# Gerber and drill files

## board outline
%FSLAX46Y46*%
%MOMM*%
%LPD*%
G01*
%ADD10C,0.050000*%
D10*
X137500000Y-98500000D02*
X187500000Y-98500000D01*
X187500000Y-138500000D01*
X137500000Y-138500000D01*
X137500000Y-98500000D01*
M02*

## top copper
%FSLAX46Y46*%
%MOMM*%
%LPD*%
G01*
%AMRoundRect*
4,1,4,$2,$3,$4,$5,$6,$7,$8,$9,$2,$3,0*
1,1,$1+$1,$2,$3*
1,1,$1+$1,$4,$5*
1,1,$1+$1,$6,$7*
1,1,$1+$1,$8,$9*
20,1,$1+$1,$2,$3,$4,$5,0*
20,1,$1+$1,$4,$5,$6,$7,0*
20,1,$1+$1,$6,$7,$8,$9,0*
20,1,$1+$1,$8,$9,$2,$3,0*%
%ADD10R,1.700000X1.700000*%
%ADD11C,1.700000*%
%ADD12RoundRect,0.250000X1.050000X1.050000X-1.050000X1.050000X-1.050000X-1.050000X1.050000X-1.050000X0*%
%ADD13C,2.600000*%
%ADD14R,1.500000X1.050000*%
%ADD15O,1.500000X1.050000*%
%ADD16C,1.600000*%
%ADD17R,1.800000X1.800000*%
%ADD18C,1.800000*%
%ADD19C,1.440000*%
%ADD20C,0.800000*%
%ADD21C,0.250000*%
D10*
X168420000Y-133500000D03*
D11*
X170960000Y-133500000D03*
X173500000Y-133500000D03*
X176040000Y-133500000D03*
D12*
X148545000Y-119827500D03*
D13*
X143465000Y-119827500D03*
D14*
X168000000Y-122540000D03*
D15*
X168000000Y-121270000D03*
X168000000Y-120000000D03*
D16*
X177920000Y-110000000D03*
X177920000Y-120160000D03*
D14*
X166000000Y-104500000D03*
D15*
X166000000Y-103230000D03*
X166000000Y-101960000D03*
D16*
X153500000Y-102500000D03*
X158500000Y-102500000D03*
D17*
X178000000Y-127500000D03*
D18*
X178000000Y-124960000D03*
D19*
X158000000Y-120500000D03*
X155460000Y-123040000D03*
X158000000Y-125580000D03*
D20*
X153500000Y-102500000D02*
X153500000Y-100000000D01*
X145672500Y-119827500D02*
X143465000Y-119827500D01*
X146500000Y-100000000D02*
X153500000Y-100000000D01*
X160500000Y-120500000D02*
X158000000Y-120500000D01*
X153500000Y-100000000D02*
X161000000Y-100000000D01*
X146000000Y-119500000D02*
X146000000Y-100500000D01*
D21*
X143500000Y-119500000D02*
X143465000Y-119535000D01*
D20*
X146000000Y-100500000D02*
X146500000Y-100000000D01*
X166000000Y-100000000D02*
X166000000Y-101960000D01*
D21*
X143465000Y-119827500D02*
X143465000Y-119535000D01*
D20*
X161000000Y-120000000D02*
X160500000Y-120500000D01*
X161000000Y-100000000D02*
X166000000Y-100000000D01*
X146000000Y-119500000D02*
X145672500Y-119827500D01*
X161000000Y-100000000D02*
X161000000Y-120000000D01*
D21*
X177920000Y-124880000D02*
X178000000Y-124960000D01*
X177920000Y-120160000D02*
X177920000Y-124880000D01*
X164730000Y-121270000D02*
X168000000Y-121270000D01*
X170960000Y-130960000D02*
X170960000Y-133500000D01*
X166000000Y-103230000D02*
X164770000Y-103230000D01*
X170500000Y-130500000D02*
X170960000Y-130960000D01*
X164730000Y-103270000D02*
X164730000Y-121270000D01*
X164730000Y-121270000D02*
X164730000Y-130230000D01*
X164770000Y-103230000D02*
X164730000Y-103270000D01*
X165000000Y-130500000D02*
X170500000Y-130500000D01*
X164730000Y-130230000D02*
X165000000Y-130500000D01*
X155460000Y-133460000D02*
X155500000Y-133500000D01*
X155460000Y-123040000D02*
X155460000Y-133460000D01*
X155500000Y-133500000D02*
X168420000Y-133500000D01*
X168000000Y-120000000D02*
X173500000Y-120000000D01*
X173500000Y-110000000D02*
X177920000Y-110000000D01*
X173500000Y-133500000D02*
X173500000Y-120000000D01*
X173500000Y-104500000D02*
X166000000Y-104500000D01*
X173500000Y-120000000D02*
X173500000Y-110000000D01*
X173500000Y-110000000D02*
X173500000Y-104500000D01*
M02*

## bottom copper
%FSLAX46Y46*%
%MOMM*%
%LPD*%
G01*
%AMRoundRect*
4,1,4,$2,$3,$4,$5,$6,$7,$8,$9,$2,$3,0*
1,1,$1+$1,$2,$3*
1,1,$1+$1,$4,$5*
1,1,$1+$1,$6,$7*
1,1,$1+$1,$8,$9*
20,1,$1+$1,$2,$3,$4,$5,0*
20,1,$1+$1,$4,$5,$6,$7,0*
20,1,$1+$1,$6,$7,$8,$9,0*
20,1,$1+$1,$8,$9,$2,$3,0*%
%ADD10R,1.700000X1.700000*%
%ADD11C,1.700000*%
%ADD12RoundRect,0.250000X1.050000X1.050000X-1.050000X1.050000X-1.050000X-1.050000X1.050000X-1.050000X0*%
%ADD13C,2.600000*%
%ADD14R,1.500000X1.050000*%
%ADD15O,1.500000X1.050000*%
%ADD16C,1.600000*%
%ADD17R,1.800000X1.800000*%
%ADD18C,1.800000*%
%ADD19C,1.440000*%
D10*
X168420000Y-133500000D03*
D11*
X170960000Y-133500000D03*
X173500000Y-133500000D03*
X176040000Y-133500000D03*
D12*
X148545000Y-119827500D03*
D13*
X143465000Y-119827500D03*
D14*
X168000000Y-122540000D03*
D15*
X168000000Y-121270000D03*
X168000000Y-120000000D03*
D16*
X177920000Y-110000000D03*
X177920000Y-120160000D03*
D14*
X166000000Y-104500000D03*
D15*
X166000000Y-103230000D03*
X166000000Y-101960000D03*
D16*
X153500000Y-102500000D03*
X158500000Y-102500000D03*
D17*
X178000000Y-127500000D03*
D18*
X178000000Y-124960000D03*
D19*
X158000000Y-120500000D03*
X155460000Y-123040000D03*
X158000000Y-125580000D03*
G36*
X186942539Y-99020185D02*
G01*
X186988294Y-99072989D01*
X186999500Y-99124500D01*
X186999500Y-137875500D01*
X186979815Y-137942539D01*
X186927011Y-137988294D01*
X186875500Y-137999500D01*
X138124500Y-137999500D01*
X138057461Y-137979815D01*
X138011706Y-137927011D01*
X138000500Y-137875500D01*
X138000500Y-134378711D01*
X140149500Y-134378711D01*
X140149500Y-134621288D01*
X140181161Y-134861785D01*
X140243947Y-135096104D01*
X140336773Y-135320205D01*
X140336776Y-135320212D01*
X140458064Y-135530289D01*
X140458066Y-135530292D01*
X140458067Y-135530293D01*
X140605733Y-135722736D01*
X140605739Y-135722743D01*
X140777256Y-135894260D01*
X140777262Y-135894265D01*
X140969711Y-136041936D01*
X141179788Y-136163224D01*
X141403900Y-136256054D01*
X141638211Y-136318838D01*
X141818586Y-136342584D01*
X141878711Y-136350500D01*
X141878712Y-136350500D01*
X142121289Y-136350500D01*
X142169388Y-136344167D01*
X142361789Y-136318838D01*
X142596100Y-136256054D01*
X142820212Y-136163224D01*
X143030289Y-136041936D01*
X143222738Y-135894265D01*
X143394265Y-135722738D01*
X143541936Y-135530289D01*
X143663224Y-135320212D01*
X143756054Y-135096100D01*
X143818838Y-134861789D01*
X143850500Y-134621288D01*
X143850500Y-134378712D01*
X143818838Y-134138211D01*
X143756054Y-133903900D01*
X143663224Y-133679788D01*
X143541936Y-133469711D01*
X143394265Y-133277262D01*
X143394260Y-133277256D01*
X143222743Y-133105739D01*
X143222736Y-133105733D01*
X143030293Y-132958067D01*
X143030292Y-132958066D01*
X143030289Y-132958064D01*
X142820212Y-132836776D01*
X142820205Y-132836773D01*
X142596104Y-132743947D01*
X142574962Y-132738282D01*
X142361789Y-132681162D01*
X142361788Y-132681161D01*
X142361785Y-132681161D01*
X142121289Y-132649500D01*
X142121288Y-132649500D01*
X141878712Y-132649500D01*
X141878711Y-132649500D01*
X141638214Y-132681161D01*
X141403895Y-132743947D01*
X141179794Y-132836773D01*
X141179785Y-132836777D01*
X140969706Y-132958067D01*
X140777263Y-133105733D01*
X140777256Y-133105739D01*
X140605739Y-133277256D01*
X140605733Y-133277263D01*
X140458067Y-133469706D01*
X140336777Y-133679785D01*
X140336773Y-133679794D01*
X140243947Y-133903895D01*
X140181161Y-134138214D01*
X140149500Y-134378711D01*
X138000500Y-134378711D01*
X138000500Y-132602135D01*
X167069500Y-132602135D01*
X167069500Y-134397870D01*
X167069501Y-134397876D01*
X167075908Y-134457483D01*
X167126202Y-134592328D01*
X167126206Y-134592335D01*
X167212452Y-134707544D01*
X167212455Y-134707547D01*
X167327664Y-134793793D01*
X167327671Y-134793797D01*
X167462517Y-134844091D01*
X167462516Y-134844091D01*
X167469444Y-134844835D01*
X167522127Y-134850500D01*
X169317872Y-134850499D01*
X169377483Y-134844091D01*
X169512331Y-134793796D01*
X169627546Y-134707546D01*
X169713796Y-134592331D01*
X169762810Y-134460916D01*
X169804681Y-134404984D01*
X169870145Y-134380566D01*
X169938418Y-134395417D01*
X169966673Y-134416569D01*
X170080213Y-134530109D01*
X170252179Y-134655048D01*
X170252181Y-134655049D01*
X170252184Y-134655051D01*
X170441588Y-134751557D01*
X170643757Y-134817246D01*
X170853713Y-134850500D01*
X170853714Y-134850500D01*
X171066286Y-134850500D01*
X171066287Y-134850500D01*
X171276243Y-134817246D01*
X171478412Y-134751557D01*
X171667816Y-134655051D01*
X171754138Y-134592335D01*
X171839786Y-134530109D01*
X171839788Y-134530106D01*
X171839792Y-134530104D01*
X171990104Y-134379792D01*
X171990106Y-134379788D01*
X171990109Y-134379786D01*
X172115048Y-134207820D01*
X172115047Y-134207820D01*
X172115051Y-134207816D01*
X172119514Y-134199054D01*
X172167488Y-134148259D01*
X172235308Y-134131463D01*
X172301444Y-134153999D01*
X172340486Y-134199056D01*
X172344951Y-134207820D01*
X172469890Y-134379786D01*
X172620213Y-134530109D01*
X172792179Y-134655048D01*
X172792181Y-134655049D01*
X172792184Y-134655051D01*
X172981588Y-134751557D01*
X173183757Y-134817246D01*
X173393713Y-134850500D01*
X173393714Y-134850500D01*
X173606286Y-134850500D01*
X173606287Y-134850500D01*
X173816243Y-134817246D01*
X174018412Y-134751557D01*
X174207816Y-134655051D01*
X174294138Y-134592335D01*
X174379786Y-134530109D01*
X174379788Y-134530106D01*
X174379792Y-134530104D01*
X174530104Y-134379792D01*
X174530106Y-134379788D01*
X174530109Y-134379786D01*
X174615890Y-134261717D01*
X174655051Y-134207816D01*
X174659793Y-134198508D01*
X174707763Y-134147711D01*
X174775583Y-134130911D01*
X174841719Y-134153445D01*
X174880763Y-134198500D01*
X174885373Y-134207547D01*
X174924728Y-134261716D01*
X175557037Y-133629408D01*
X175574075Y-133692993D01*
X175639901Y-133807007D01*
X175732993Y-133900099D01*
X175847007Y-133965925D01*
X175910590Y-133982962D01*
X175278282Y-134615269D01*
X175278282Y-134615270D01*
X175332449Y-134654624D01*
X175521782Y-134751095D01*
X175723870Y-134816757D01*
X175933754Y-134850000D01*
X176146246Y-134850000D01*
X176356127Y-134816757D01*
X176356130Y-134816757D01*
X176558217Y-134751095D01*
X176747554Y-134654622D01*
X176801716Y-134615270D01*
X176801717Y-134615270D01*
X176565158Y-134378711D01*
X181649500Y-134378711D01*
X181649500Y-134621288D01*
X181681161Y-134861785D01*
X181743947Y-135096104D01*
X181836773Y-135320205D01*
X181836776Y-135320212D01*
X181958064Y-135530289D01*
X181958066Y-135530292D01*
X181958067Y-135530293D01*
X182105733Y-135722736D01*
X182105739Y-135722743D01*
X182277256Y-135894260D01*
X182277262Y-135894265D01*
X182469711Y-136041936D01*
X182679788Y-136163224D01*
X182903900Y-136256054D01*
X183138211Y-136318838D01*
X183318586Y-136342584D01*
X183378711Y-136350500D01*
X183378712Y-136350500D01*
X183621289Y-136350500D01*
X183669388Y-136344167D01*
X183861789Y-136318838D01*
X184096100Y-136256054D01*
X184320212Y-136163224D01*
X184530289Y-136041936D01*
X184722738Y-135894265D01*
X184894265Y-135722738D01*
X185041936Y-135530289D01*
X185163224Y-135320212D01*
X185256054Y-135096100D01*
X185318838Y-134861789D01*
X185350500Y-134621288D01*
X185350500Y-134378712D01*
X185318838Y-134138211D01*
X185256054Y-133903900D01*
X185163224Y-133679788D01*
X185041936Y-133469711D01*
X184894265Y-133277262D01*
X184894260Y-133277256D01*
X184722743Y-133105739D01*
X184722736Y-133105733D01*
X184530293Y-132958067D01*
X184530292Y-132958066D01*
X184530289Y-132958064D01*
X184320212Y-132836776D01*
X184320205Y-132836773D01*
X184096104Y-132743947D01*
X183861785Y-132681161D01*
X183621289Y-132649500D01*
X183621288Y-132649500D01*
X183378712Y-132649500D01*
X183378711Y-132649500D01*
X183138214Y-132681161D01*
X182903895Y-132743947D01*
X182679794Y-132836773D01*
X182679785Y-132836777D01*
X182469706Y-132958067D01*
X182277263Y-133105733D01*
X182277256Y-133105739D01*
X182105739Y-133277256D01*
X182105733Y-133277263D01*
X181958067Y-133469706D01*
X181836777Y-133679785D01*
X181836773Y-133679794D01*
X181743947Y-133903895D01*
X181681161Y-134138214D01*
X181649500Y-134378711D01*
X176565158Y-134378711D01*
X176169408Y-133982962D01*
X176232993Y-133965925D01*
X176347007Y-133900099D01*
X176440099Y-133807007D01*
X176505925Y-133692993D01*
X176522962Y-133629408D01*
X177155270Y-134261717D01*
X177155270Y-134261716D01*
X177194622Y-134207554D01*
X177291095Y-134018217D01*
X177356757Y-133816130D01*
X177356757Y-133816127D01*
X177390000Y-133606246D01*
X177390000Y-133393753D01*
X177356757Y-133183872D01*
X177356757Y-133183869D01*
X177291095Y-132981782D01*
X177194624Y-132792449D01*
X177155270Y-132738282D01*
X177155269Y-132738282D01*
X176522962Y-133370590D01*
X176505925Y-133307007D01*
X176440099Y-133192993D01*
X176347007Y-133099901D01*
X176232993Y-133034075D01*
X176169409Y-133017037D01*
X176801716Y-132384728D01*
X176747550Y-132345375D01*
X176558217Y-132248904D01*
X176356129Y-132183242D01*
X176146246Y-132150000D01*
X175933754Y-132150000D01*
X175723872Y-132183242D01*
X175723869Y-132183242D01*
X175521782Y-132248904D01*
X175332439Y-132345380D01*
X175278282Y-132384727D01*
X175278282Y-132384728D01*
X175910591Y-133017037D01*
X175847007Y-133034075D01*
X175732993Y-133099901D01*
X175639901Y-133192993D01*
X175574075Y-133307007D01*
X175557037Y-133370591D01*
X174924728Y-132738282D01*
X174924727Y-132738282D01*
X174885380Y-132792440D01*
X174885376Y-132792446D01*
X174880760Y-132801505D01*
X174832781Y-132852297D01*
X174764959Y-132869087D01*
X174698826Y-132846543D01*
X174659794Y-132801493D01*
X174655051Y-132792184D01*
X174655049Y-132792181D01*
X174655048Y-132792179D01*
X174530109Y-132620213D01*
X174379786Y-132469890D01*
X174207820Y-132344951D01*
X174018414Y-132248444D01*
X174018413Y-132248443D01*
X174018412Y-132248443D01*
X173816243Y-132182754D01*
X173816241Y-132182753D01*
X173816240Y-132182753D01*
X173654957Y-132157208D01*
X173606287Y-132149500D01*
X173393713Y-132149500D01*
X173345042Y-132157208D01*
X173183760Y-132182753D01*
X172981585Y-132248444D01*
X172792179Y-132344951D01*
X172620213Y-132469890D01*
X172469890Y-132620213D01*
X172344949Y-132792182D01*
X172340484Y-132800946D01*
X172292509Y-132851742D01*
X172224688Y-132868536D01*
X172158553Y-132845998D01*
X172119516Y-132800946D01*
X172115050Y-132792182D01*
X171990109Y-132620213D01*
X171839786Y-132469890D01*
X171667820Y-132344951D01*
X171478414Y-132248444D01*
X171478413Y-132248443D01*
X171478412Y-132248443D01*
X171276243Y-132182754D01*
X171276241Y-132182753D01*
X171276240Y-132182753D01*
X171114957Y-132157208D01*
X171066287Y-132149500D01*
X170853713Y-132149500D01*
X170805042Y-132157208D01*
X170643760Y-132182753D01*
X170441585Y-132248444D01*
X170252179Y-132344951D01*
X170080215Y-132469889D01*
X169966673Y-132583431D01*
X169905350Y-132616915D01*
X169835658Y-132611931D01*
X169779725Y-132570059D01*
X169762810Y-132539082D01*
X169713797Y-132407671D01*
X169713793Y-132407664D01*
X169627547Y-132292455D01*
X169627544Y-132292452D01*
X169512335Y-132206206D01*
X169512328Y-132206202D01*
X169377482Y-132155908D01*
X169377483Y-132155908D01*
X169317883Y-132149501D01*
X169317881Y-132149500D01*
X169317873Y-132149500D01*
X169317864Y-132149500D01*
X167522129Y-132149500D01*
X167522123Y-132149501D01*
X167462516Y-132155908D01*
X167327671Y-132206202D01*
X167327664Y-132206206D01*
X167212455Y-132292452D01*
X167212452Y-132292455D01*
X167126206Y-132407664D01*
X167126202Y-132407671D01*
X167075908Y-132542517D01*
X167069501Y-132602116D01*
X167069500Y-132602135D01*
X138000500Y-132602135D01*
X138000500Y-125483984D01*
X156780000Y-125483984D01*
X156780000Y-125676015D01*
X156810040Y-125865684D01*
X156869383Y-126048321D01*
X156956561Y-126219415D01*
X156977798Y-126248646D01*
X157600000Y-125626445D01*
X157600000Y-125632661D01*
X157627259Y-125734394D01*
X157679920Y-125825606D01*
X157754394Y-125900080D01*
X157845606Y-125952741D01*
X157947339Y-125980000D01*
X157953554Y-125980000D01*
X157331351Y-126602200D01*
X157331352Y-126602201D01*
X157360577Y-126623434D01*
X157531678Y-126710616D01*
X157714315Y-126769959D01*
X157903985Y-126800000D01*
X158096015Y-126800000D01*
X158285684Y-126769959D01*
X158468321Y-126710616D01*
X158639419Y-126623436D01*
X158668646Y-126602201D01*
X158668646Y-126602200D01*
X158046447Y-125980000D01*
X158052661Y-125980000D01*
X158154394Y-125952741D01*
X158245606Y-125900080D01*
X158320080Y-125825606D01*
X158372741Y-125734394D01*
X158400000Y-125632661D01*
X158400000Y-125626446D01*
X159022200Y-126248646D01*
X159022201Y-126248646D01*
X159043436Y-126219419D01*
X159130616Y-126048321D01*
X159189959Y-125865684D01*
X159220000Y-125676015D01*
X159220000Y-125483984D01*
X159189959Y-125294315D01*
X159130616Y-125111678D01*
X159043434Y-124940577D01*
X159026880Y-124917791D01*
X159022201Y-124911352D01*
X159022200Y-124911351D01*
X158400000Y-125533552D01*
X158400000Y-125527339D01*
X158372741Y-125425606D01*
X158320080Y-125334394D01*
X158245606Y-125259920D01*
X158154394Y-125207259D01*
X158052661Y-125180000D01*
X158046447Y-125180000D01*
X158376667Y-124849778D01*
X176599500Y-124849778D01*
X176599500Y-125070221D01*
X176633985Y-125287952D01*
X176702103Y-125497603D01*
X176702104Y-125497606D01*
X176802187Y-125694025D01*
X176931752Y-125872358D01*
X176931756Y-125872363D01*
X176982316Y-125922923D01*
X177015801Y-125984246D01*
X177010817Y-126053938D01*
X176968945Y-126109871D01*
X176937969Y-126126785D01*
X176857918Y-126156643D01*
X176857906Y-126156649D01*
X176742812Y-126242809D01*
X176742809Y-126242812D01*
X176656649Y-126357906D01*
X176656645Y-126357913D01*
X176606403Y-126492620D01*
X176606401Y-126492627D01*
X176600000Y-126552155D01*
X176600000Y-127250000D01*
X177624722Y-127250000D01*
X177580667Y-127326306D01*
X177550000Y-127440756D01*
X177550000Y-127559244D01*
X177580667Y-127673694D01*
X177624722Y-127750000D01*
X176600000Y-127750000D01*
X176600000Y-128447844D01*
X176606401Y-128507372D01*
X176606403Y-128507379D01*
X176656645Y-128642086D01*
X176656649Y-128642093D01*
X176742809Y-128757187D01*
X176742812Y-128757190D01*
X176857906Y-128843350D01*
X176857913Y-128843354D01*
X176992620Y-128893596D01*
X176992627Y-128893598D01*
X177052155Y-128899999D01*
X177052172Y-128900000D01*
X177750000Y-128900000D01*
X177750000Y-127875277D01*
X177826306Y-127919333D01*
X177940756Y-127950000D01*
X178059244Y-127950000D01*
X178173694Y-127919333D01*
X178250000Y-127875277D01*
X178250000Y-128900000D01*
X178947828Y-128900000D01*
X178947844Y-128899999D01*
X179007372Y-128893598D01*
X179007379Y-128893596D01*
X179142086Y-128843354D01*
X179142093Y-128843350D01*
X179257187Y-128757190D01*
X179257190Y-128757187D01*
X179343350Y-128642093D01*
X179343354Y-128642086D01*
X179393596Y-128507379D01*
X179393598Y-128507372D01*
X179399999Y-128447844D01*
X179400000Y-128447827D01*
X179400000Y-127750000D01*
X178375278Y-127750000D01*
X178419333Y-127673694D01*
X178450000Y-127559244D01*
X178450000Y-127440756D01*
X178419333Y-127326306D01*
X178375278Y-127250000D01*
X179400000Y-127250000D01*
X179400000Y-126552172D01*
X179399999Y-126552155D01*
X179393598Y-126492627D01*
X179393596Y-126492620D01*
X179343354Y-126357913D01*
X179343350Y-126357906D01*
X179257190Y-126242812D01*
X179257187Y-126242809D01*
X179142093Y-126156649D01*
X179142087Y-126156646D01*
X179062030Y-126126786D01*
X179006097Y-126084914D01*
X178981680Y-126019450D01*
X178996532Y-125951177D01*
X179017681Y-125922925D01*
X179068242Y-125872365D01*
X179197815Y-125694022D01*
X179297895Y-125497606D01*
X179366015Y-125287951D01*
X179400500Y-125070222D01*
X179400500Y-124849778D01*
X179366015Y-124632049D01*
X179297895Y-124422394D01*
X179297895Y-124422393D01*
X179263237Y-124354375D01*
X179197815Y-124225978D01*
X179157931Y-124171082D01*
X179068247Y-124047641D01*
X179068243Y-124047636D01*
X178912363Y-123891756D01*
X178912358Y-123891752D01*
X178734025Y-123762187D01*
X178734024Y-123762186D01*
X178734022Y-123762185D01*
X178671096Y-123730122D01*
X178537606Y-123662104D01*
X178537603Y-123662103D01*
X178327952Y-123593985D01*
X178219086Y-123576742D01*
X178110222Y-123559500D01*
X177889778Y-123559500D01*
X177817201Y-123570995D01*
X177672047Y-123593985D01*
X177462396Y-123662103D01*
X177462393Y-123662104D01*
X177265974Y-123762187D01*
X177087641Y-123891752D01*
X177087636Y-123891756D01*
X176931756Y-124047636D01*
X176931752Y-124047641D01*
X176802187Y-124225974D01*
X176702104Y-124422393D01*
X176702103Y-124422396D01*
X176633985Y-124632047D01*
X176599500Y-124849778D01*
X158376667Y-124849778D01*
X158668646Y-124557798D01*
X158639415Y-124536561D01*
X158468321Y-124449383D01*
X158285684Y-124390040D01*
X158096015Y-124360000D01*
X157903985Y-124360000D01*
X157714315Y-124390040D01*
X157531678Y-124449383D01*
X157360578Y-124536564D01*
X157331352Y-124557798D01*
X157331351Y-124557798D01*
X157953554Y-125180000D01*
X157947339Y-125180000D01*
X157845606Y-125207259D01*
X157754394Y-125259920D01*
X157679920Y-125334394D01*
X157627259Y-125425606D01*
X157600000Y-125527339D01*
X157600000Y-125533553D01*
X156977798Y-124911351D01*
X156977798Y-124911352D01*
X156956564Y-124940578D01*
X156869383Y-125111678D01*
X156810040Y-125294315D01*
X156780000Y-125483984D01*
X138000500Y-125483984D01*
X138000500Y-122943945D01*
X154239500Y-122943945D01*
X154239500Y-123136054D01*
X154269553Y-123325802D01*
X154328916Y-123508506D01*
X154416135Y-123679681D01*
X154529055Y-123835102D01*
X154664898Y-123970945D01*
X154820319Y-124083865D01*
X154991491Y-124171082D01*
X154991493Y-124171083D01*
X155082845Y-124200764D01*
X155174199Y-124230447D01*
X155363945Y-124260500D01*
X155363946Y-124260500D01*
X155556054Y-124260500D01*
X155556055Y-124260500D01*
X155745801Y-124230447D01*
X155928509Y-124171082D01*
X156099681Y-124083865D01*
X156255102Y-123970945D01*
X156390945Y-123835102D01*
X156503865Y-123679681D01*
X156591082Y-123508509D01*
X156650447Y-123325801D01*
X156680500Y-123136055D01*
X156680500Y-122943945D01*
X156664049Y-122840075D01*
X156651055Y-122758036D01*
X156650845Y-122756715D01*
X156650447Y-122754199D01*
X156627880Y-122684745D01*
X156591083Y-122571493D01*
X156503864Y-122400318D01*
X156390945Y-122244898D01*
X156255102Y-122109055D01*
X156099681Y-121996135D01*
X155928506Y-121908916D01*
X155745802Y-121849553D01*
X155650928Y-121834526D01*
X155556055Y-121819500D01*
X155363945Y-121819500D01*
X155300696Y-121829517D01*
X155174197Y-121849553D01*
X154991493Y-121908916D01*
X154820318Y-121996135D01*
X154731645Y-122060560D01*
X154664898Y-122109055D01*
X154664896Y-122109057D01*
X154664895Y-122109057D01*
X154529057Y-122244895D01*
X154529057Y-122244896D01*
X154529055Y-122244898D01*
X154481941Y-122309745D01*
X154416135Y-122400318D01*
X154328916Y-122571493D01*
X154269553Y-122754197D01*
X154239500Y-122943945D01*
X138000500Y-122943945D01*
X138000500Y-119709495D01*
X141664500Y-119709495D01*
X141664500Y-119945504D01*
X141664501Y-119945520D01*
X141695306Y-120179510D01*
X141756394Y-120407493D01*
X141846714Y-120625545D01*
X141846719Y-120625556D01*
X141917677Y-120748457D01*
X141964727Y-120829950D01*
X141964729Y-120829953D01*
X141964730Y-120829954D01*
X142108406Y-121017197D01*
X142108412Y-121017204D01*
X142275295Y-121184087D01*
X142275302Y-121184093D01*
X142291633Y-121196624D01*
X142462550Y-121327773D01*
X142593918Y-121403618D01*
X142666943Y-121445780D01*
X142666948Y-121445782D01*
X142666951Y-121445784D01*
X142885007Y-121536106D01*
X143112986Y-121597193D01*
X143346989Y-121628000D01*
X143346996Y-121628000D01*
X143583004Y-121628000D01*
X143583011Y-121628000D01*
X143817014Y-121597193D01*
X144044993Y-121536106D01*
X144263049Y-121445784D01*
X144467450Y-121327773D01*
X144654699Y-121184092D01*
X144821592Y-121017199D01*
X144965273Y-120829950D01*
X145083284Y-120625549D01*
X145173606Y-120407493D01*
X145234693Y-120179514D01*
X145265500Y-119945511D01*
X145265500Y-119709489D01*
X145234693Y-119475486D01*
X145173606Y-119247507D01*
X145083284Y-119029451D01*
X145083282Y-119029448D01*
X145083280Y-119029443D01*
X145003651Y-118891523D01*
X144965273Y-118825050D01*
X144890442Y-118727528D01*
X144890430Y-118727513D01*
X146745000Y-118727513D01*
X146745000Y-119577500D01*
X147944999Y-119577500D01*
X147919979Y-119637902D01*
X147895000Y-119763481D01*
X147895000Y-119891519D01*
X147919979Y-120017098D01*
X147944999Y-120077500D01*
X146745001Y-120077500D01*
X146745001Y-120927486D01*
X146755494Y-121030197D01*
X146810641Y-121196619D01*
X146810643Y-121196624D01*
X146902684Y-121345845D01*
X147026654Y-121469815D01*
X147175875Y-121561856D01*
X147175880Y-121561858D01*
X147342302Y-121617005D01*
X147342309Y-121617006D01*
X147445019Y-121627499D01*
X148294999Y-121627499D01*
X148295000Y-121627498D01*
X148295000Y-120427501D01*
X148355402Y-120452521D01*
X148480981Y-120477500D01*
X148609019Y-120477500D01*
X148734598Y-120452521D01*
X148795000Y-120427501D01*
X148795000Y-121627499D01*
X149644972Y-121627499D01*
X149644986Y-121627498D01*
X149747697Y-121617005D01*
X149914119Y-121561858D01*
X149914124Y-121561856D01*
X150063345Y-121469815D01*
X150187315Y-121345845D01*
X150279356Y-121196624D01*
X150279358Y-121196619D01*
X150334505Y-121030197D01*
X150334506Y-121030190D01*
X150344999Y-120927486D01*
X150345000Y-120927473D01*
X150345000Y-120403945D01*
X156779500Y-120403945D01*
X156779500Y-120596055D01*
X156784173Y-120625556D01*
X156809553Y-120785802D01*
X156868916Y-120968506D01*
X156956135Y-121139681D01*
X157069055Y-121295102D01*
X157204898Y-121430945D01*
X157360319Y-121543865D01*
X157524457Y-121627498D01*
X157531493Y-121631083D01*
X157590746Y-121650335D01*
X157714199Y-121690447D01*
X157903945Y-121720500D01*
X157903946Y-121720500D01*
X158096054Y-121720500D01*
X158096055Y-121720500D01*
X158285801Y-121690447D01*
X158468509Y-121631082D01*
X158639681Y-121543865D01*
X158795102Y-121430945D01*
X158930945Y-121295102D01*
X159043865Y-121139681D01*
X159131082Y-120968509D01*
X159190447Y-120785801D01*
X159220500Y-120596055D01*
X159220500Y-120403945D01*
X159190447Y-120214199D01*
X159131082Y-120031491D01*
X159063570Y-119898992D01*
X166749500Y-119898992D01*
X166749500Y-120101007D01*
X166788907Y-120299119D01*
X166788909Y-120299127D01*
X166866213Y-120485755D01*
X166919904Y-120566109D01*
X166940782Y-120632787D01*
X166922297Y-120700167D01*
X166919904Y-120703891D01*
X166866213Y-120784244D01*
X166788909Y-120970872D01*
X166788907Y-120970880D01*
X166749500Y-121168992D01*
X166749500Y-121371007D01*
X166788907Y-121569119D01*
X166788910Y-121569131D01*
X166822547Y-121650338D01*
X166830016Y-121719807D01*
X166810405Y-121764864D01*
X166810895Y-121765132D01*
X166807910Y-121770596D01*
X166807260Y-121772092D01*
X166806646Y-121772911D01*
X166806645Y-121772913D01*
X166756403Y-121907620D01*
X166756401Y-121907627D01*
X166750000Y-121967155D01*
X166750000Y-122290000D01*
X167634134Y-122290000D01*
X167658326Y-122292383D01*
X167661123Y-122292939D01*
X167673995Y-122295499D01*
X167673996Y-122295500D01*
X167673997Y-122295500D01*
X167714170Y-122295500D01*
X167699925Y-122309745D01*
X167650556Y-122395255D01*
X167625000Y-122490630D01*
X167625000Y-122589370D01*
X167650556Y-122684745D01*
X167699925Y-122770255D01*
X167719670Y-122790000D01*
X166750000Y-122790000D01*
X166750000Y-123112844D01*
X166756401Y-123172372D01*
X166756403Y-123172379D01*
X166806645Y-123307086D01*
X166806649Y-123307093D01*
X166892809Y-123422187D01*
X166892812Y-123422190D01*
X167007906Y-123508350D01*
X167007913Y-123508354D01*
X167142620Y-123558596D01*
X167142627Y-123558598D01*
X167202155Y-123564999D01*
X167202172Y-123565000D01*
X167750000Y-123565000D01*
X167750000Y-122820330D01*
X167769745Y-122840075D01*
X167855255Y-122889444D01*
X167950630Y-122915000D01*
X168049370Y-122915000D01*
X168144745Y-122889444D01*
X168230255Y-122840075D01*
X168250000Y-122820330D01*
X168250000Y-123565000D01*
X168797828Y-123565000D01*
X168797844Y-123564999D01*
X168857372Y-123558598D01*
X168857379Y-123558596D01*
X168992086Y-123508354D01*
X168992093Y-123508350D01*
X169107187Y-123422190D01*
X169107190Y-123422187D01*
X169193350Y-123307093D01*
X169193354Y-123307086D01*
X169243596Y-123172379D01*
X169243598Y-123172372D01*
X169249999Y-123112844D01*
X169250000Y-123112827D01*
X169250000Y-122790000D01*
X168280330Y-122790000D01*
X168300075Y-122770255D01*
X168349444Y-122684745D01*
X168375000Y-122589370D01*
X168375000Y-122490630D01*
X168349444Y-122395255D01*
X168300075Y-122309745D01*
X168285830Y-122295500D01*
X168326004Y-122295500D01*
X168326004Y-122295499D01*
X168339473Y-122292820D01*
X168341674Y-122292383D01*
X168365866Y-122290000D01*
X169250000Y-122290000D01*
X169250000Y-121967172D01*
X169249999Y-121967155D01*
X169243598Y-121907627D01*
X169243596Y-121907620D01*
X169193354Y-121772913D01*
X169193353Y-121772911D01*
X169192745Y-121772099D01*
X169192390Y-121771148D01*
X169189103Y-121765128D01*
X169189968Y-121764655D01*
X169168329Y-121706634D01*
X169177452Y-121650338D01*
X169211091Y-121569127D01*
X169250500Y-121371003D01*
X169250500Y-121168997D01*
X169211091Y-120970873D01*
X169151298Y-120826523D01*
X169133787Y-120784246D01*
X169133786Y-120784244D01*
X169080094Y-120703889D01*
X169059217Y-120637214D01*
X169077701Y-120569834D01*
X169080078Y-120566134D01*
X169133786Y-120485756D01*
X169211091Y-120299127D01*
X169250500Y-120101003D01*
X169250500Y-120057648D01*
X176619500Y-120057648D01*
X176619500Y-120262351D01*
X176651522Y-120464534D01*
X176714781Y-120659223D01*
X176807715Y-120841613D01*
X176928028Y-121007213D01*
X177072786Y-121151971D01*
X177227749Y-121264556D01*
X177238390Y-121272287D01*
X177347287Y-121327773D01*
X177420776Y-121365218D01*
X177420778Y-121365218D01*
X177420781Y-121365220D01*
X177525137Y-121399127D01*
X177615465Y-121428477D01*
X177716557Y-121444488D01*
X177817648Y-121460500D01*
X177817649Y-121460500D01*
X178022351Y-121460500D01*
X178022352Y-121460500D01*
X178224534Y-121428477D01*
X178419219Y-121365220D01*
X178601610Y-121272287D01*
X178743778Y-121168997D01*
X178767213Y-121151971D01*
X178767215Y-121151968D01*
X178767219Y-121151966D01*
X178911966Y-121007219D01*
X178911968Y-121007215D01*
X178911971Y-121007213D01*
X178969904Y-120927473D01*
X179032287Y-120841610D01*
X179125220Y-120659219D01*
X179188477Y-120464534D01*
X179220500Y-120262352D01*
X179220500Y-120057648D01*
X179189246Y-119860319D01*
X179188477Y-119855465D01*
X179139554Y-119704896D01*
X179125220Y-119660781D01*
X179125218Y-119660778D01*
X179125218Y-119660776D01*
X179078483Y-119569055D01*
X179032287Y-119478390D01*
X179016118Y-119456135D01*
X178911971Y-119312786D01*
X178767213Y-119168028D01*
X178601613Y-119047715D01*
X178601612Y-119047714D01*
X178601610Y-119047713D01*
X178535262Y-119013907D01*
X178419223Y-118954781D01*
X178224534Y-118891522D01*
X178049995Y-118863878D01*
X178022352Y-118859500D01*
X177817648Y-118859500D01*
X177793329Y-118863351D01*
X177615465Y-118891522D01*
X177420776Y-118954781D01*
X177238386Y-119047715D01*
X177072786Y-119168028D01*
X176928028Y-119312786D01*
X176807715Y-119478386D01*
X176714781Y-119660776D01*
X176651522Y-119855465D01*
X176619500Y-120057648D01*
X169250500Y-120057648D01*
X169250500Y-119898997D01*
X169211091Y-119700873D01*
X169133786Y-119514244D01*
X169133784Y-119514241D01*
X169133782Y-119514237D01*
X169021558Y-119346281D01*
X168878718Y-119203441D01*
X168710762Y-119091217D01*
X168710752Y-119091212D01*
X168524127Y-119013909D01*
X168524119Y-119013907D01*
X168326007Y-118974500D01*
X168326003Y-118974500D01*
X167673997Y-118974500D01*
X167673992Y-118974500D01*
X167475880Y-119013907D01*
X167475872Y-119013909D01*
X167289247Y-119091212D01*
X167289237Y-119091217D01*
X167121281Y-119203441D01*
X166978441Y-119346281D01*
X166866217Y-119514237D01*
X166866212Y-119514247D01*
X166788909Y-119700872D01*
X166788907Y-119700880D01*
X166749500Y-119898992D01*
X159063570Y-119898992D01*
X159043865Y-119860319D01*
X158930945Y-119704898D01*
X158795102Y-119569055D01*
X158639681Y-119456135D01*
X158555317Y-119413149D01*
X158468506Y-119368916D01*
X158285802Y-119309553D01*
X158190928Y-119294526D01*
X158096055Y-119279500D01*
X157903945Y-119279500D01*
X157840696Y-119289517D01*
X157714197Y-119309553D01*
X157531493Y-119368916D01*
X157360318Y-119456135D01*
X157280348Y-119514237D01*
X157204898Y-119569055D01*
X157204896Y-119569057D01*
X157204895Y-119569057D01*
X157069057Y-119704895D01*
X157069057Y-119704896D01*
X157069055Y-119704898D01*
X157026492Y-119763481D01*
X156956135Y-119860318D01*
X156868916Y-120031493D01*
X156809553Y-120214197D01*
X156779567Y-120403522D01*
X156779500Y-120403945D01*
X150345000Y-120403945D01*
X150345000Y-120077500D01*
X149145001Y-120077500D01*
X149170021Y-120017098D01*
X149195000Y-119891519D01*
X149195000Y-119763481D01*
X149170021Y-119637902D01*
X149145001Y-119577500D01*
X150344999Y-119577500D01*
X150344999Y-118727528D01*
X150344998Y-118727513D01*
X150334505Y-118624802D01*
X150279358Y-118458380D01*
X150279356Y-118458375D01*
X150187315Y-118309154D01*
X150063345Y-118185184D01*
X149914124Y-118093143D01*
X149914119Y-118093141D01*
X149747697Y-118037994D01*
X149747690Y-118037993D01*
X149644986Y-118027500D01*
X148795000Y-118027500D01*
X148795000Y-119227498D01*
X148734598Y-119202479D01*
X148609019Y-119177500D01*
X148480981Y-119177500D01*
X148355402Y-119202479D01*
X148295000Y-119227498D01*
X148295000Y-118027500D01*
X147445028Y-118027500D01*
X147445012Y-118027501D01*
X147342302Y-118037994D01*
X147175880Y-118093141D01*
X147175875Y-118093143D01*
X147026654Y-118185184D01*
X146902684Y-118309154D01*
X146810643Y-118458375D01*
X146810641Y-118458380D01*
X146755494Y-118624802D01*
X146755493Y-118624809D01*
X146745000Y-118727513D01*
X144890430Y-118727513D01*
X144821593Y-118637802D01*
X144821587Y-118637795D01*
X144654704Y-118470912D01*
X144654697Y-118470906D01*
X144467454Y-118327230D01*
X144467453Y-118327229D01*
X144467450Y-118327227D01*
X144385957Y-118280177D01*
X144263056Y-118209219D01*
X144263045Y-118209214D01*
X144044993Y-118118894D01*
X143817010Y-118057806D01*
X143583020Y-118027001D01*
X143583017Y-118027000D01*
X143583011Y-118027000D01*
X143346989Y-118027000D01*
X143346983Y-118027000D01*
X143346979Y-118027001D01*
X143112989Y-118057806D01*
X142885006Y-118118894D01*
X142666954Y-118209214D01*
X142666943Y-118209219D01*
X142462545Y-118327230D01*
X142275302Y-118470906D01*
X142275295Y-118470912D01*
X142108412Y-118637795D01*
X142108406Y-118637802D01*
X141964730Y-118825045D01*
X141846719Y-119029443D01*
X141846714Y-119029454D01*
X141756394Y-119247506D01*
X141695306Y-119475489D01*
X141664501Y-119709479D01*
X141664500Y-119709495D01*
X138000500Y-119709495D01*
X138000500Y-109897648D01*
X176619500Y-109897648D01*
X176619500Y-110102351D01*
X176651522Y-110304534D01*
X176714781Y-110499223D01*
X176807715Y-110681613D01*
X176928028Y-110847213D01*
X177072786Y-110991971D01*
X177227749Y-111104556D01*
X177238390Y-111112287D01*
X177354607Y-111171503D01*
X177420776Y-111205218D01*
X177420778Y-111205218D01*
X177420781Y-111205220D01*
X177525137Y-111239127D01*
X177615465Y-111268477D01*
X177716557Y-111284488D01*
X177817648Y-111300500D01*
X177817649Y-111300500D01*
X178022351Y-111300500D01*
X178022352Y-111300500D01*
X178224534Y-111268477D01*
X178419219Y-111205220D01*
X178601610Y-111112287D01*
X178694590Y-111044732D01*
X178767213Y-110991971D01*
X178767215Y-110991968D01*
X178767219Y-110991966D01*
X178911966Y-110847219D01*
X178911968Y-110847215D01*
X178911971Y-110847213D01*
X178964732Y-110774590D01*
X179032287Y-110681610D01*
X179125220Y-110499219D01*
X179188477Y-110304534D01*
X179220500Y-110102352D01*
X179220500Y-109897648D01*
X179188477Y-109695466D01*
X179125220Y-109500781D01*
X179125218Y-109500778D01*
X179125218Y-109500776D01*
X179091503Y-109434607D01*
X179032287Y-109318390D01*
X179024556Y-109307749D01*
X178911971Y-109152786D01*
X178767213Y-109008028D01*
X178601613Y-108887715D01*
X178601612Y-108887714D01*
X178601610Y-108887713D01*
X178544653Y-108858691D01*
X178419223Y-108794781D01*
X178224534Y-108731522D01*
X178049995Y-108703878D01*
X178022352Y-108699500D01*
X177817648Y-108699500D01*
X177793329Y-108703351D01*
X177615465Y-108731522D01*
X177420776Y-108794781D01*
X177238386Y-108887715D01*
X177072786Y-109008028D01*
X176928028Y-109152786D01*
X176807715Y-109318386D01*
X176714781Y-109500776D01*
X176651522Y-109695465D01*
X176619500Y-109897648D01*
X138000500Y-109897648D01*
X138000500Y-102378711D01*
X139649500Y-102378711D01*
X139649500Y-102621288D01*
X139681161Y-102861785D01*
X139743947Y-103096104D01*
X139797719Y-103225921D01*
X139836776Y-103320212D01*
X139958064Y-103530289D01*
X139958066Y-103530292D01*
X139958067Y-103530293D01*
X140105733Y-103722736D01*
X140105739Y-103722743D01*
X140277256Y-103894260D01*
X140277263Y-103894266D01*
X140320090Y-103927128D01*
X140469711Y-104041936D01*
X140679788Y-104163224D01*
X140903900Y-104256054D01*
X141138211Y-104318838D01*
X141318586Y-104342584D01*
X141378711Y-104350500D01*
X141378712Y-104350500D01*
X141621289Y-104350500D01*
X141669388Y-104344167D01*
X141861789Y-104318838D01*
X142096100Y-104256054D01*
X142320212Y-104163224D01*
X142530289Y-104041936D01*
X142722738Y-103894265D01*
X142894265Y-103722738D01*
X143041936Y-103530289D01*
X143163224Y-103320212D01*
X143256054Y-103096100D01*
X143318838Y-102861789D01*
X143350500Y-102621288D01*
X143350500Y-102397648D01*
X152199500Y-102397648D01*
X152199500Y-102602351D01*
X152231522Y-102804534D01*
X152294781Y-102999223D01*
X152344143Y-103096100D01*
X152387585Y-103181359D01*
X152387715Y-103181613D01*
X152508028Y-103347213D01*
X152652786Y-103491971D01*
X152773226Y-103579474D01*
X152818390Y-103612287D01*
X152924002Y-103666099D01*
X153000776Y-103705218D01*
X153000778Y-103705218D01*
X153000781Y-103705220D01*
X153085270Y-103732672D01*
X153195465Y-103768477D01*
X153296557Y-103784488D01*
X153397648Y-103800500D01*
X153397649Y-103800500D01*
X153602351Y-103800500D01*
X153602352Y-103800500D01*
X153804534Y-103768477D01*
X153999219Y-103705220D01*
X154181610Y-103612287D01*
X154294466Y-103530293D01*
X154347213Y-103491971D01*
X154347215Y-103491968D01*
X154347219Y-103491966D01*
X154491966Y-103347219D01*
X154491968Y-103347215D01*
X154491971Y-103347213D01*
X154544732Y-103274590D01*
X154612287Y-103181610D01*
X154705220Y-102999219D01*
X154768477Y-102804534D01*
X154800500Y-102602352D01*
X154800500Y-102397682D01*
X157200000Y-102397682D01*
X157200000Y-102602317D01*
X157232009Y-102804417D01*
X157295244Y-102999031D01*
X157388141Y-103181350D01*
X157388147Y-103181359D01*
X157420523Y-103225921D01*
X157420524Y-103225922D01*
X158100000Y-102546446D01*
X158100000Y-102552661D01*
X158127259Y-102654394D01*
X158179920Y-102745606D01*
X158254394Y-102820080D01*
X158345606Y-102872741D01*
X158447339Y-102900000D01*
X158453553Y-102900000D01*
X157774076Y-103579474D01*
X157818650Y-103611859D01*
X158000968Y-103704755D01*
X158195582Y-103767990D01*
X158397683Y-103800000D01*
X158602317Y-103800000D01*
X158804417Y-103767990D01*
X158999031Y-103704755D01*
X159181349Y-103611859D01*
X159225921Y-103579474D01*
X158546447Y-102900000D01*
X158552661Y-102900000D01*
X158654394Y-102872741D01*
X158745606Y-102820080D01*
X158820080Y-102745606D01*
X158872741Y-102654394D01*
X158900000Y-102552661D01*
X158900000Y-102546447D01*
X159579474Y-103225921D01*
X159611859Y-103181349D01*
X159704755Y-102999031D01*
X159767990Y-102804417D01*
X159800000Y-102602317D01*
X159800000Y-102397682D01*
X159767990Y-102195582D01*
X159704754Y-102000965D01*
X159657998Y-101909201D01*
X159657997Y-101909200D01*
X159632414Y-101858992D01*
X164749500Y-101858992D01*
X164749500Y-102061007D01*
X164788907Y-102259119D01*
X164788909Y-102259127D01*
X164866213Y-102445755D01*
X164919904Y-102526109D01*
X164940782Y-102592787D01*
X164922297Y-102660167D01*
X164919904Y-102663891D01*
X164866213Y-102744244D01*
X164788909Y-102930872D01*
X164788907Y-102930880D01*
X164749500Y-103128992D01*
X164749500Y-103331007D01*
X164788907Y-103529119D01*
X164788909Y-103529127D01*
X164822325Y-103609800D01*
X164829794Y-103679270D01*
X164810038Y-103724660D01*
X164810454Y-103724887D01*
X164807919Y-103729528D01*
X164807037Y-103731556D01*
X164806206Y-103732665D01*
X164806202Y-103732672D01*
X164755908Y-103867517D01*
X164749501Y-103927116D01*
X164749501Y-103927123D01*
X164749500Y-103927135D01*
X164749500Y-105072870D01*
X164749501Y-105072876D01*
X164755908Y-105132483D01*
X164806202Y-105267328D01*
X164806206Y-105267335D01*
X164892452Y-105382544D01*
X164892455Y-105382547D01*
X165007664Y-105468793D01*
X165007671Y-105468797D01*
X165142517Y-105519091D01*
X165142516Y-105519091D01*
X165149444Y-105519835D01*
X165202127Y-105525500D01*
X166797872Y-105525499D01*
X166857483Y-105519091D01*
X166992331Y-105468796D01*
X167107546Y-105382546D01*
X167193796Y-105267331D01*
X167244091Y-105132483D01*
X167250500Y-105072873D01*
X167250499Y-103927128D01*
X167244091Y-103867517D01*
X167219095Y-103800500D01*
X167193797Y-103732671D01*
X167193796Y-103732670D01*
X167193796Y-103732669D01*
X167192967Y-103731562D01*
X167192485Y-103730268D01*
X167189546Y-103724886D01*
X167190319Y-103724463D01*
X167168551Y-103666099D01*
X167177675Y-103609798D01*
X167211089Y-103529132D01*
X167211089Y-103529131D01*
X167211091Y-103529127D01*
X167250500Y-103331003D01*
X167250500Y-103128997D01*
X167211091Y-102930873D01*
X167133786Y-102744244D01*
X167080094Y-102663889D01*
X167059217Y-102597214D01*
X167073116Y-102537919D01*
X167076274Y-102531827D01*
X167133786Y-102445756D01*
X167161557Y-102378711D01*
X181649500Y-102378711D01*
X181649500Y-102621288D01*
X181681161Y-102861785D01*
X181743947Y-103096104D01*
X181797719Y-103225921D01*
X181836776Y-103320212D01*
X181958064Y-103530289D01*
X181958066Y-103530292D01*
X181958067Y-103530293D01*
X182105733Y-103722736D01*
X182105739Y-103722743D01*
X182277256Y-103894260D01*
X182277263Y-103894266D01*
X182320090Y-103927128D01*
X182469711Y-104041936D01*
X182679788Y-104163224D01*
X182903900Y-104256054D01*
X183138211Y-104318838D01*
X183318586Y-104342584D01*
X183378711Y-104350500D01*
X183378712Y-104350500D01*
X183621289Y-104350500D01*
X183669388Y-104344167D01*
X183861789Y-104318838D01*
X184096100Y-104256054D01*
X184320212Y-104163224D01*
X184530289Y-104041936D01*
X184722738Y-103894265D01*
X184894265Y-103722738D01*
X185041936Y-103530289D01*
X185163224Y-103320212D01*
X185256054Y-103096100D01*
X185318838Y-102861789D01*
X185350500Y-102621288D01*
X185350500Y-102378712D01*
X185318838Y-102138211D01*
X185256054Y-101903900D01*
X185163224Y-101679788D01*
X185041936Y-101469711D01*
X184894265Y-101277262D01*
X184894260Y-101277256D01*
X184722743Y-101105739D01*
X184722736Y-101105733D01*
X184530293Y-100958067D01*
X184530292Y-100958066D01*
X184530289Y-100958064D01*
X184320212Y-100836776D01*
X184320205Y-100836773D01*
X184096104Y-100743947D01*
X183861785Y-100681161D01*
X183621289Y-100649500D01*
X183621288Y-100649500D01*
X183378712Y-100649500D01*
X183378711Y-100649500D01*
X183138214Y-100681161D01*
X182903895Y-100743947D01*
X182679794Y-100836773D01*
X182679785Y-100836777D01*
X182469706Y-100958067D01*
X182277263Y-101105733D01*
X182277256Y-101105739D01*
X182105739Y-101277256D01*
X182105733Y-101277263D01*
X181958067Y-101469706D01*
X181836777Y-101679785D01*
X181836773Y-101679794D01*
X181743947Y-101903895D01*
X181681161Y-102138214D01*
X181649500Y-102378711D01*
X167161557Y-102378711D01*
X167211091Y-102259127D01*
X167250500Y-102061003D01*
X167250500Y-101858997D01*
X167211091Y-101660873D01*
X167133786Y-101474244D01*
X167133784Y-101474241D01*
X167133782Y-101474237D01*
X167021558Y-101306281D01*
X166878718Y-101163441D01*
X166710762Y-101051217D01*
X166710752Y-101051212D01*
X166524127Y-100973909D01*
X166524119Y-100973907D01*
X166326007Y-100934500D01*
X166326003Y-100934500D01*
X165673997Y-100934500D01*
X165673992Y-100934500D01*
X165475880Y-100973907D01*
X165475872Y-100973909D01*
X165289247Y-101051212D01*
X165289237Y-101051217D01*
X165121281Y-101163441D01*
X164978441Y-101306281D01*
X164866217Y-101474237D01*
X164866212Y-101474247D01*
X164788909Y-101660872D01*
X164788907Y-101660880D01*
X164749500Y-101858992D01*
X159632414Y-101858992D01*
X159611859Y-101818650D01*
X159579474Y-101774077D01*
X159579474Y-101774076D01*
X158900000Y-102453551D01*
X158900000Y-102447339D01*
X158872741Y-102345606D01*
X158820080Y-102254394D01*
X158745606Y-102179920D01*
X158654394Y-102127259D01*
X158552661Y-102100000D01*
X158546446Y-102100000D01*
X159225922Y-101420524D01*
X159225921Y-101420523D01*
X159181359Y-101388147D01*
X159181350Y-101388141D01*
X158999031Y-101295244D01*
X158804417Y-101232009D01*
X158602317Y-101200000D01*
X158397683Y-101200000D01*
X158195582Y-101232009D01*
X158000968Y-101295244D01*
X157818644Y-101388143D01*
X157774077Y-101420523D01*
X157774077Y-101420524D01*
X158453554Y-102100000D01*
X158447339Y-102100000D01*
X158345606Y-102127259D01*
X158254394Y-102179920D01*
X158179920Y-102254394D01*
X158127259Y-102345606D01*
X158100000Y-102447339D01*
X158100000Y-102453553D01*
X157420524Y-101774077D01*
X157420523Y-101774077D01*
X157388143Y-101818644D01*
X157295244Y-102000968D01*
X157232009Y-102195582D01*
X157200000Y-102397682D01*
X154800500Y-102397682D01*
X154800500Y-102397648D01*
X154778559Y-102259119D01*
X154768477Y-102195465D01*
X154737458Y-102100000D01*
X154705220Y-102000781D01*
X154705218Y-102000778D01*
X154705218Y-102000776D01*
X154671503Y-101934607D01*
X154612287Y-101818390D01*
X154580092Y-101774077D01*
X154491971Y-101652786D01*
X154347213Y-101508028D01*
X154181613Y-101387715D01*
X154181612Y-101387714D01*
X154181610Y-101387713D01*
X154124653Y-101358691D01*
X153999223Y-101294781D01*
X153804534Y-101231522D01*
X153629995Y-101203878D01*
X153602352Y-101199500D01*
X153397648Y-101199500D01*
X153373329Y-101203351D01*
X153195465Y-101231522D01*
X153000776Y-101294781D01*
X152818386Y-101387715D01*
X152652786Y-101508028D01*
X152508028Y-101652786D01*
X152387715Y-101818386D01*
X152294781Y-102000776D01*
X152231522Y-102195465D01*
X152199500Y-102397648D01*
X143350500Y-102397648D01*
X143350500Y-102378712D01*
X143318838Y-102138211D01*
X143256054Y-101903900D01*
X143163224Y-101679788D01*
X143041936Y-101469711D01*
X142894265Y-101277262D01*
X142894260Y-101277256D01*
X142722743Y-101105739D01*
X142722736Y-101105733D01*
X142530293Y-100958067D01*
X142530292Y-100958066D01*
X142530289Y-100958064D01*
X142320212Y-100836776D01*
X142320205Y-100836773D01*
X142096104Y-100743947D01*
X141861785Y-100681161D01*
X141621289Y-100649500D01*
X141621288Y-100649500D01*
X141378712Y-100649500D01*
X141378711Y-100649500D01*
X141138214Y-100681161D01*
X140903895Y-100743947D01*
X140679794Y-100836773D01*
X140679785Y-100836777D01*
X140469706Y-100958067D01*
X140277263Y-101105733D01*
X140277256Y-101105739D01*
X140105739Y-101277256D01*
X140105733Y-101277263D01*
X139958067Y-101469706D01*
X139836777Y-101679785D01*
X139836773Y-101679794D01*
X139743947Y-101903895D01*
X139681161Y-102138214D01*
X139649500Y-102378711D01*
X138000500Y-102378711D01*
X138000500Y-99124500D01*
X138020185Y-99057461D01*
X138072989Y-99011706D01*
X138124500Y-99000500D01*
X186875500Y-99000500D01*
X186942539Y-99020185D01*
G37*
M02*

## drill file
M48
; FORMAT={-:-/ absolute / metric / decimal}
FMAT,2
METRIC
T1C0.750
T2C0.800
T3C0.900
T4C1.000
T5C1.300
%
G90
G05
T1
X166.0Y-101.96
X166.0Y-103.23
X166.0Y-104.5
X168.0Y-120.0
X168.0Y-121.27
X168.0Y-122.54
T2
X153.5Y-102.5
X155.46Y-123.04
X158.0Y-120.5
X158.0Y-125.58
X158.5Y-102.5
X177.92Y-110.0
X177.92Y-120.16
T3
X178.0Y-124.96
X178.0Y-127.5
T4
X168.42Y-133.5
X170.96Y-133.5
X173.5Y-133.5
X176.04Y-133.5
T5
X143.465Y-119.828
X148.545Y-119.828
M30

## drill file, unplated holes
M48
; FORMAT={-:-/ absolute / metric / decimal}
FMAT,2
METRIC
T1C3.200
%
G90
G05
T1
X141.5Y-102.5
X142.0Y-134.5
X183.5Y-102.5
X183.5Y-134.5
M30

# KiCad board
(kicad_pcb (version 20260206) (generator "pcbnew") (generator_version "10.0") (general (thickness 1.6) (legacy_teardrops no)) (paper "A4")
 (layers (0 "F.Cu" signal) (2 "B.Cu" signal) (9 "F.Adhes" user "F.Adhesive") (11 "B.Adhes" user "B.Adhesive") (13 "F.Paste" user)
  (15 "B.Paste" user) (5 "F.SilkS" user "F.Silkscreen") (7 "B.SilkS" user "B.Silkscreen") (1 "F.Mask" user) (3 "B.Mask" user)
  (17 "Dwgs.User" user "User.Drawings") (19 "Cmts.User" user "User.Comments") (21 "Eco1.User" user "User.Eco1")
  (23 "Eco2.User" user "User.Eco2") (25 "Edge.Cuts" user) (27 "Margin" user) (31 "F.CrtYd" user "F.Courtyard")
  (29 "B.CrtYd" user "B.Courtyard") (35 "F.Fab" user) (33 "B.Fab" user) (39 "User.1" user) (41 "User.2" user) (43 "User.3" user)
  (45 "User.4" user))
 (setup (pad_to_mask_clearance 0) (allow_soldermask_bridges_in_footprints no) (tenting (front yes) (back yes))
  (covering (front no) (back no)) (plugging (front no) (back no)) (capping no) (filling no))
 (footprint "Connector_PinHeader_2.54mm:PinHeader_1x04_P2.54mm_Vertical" (layer "F.Cu") (at 168.42 133.5 90)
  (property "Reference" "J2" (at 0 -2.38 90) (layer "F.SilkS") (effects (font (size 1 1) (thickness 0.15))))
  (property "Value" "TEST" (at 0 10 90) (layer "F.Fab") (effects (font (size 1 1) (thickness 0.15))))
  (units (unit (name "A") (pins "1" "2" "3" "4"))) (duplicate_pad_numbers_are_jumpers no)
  (pad "1" thru_hole rect (at 0 0 90) (size 1.7 1.7) (drill 1) (layers "*.Cu" "*.Mask") (remove_unused_layers no) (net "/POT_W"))
  (pad "2" thru_hole circle (at 0 2.54 90) (size 1.7 1.7) (drill 1) (layers "*.Cu" "*.Mask") (remove_unused_layers no) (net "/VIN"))
  (pad "3" thru_hole circle (at 0 5.08 90) (size 1.7 1.7) (drill 1) (layers "*.Cu" "*.Mask") (remove_unused_layers no) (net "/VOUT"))
  (pad "4" thru_hole circle (at 0 7.62 90) (size 1.7 1.7) (drill 1) (layers "*.Cu" "*.Mask") (remove_unused_layers no) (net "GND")))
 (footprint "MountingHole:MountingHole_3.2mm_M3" (layer "F.Cu") (at 141.5 102.5)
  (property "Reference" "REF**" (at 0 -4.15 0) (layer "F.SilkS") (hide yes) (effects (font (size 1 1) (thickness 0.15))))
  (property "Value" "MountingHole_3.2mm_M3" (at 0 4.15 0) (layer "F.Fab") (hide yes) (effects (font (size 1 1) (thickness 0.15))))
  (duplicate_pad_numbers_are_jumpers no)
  (pad "" np_thru_hole circle (at 0 0) (size 3.2 3.2) (drill 3.2) (layers "*.Cu" "*.Mask")))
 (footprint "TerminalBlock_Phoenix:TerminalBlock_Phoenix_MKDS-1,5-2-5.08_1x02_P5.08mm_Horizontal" (layer "F.Cu") (at 148.545 119.8275 180)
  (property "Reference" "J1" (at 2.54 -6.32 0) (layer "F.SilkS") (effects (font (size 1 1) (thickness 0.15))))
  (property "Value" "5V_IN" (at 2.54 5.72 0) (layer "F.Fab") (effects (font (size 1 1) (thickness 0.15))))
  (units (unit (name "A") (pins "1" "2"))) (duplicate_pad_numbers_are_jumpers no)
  (pad "1" thru_hole roundrect (at 0 0 180) (size 2.6 2.6) (drill 1.3) (layers "*.Cu" "*.Mask") (remove_unused_layers no)
   (roundrect_rratio 0.096154) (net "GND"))
  (pad "2" thru_hole circle (at 5.08 0 180) (size 2.6 2.6) (drill 1.3) (layers "*.Cu" "*.Mask") (remove_unused_layers no) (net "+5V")))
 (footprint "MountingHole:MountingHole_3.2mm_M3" (layer "F.Cu") (at 183.5 102.5)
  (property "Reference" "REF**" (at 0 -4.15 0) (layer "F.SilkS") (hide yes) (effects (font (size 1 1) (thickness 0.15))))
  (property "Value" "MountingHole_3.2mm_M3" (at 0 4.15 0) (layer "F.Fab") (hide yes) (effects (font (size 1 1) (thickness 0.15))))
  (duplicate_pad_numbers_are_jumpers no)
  (pad "" np_thru_hole circle (at 0 0) (size 3.2 3.2) (drill 3.2) (layers "*.Cu" "*.Mask")))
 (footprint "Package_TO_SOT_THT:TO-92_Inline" (layer "F.Cu") (at 168 122.54 90)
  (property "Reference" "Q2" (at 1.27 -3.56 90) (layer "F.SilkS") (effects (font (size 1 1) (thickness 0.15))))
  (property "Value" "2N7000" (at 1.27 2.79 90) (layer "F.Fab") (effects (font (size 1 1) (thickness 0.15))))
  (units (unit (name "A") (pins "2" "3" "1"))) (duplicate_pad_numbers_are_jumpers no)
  (pad "1" thru_hole rect (at 0 0 90) (size 1.05 1.5) (drill 0.75) (layers "*.Cu" "*.Mask") (remove_unused_layers no) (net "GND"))
  (pad "2" thru_hole oval (at 1.27 0 90) (size 1.05 1.5) (drill 0.75) (layers "*.Cu" "*.Mask") (remove_unused_layers no) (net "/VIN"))
  (pad "3" thru_hole oval (at 2.54 0 90) (size 1.05 1.5) (drill 0.75) (layers "*.Cu" "*.Mask") (remove_unused_layers no) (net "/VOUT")))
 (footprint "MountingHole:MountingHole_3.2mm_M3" (layer "F.Cu") (at 142 134.5)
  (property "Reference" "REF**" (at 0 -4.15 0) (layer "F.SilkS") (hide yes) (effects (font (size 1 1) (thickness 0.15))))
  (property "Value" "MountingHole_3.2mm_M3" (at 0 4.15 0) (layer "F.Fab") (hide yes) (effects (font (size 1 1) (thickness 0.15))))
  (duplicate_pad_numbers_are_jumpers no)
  (pad "" np_thru_hole circle (at 0 0) (size 3.2 3.2) (drill 3.2) (layers "*.Cu" "*.Mask")))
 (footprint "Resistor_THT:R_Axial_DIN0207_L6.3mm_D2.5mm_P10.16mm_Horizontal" (layer "F.Cu") (at 177.92 110 -90)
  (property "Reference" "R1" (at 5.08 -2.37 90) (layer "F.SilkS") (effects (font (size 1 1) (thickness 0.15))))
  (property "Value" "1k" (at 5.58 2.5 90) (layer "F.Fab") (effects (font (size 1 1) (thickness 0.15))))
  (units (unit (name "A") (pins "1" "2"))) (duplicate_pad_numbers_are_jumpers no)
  (pad "1" thru_hole circle (at 0 0 270) (size 1.6 1.6) (drill 0.8) (layers "*.Cu" "*.Mask") (remove_unused_layers no) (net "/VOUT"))
  (pad "2" thru_hole circle (at 10.16 0 270) (size 1.6 1.6) (drill 0.8) (layers "*.Cu" "*.Mask") (remove_unused_layers no)
   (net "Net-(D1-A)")))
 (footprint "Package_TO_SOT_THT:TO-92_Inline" (layer "F.Cu") (at 166 104.5 90)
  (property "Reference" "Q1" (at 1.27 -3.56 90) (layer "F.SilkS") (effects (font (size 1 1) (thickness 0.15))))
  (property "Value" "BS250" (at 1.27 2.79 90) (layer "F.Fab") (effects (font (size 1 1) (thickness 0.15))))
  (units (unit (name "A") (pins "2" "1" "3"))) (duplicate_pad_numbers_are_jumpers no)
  (pad "1" thru_hole rect (at 0 0 90) (size 1.05 1.5) (drill 0.75) (layers "*.Cu" "*.Mask") (remove_unused_layers no) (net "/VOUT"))
  (pad "2" thru_hole oval (at 1.27 0 90) (size 1.05 1.5) (drill 0.75) (layers "*.Cu" "*.Mask") (remove_unused_layers no) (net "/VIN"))
  (pad "3" thru_hole oval (at 2.54 0 90) (size 1.05 1.5) (drill 0.75) (layers "*.Cu" "*.Mask") (remove_unused_layers no) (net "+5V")))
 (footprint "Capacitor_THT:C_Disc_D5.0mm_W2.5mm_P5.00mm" (layer "F.Cu") (at 153.5 102.5)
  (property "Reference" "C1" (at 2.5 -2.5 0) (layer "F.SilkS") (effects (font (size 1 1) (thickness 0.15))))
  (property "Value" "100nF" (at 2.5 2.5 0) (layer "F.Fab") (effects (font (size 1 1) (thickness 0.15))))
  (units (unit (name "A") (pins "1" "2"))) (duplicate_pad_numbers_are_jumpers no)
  (pad "1" thru_hole circle (at 0 0) (size 1.6 1.6) (drill 0.8) (layers "*.Cu" "*.Mask") (remove_unused_layers no) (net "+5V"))
  (pad "2" thru_hole circle (at 5 0) (size 1.6 1.6) (drill 0.8) (layers "*.Cu" "*.Mask") (remove_unused_layers no) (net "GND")))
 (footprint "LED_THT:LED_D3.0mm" (layer "F.Cu") (at 178 127.5 90)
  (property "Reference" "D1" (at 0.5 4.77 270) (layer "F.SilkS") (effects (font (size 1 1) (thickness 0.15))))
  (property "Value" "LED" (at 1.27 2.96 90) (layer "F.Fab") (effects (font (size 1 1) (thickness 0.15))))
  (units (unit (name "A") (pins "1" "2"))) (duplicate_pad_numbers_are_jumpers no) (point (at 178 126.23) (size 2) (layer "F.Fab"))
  (pad "1" thru_hole rect (at 0 0 90) (size 1.8 1.8) (drill 0.9) (layers "*.Cu" "*.Mask") (remove_unused_layers no) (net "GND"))
  (pad "2" thru_hole circle (at 2.54 0 90) (size 1.8 1.8) (drill 0.9) (layers "*.Cu" "*.Mask") (remove_unused_layers no) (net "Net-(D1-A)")))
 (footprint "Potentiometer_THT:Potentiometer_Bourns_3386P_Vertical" (layer "F.Cu") (at 158 120.5 180)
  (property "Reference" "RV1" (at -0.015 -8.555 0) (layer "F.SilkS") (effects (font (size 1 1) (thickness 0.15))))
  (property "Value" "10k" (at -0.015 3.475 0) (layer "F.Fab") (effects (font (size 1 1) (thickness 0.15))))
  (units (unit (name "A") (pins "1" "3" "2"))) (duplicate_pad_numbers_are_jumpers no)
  (pad "1" thru_hole circle (at 0 0 180) (size 1.44 1.44) (drill 0.8) (layers "*.Cu" "*.Mask") (remove_unused_layers no) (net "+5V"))
  (pad "2" thru_hole circle (at 2.54 -2.54 180) (size 1.44 1.44) (drill 0.8) (layers "*.Cu" "*.Mask") (remove_unused_layers no)
   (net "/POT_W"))
  (pad "3" thru_hole circle (at 0 -5.08 180) (size 1.44 1.44) (drill 0.8) (layers "*.Cu" "*.Mask") (remove_unused_layers no) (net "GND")))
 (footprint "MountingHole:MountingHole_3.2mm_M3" (layer "F.Cu") (at 183.5 134.5)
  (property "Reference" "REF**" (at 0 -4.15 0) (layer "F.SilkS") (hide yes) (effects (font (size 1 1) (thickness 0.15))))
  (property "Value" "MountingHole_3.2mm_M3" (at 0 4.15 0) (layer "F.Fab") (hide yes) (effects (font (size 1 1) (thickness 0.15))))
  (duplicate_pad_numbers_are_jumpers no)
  (pad "" np_thru_hole circle (at 0 0) (size 3.2 3.2) (drill 3.2) (layers "*.Cu" "*.Mask")))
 (gr_rect (start 137.5 98.5) (end 187.5 138.5) (stroke (width 0.05) (type default)) (fill no) (layer "Edge.Cuts"))
 (segment (start 155.46 133.46) (end 155.5 133.5) (width 0.25) (layer "F.Cu") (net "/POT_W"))
 (segment (start 155.46 123.04) (end 155.46 133.46) (width 0.25) (layer "F.Cu") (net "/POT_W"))
 (segment (start 155.5 133.5) (end 168.42 133.5) (width 0.25) (layer "F.Cu") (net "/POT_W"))
 (segment (start 164.73 121.27) (end 168 121.27) (width 0.25) (layer "F.Cu") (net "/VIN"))
 (segment (start 170.96 130.96) (end 170.96 133.5) (width 0.25) (layer "F.Cu") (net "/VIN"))
 (segment (start 166 103.23) (end 164.77 103.23) (width 0.25) (layer "F.Cu") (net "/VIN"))
 (segment (start 170.5 130.5) (end 170.96 130.96) (width 0.25) (layer "F.Cu") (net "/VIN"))
 (segment (start 164.73 103.27) (end 164.73 121.27) (width 0.25) (layer "F.Cu") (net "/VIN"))
 (segment (start 164.73 121.27) (end 164.73 130.23) (width 0.25) (layer "F.Cu") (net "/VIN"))
 (segment (start 164.77 103.23) (end 164.73 103.27) (width 0.25) (layer "F.Cu") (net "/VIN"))
 (segment (start 165 130.5) (end 170.5 130.5) (width 0.25) (layer "F.Cu") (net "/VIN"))
 (segment (start 164.73 130.23) (end 165 130.5) (width 0.25) (layer "F.Cu") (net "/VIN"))
 (segment (start 168 120) (end 173.5 120) (width 0.25) (layer "F.Cu") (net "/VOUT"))
 (segment (start 173.5 110) (end 177.92 110) (width 0.25) (layer "F.Cu") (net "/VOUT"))
 (segment (start 173.5 133.5) (end 173.5 120) (width 0.25) (layer "F.Cu") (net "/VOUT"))
 (segment (start 173.5 104.5) (end 166 104.5) (width 0.25) (layer "F.Cu") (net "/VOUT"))
 (segment (start 173.5 120) (end 173.5 110) (width 0.25) (layer "F.Cu") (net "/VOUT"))
 (segment (start 173.5 110) (end 173.5 104.5) (width 0.25) (layer "F.Cu") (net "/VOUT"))
 (segment (start 153.5 102.5) (end 153.5 100) (width 0.8) (layer "F.Cu") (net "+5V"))
 (segment (start 145.6725 119.8275) (end 143.465 119.8275) (width 0.8) (layer "F.Cu") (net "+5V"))
 (segment (start 146.5 100) (end 153.5 100) (width 0.8) (layer "F.Cu") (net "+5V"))
 (segment (start 160.5 120.5) (end 158 120.5) (width 0.8) (layer "F.Cu") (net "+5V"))
 (segment (start 153.5 100) (end 161 100) (width 0.8) (layer "F.Cu") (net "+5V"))
 (segment (start 146 119.5) (end 146 100.5) (width 0.8) (layer "F.Cu") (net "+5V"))
 (segment (start 143.5 119.5) (end 143.465 119.535) (width 0.25) (layer "F.Cu") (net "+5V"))
 (segment (start 146 100.5) (end 146.5 100) (width 0.8) (layer "F.Cu") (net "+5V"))
 (segment (start 166 100) (end 166 101.96) (width 0.8) (layer "F.Cu") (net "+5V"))
 (segment (start 143.465 119.8275) (end 143.465 119.535) (width 0.25) (layer "F.Cu") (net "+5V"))
 (segment (start 161 120) (end 160.5 120.5) (width 0.8) (layer "F.Cu") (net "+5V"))
 (segment (start 161 100) (end 166 100) (width 0.8) (layer "F.Cu") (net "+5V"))
 (segment (start 146 119.5) (end 145.6725 119.8275) (width 0.8) (layer "F.Cu") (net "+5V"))
 (segment (start 161 100) (end 161 120) (width 0.8) (layer "F.Cu") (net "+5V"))
 (segment (start 177.92 124.88) (end 178 124.96) (width 0.25) (layer "F.Cu") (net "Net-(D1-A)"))
 (segment (start 177.92 120.16) (end 177.92 124.88) (width 0.25) (layer "F.Cu") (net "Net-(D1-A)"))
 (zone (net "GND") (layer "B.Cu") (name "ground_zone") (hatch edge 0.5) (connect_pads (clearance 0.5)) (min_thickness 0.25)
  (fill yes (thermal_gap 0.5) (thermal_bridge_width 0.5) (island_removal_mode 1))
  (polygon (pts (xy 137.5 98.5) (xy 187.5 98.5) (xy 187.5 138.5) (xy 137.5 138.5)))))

